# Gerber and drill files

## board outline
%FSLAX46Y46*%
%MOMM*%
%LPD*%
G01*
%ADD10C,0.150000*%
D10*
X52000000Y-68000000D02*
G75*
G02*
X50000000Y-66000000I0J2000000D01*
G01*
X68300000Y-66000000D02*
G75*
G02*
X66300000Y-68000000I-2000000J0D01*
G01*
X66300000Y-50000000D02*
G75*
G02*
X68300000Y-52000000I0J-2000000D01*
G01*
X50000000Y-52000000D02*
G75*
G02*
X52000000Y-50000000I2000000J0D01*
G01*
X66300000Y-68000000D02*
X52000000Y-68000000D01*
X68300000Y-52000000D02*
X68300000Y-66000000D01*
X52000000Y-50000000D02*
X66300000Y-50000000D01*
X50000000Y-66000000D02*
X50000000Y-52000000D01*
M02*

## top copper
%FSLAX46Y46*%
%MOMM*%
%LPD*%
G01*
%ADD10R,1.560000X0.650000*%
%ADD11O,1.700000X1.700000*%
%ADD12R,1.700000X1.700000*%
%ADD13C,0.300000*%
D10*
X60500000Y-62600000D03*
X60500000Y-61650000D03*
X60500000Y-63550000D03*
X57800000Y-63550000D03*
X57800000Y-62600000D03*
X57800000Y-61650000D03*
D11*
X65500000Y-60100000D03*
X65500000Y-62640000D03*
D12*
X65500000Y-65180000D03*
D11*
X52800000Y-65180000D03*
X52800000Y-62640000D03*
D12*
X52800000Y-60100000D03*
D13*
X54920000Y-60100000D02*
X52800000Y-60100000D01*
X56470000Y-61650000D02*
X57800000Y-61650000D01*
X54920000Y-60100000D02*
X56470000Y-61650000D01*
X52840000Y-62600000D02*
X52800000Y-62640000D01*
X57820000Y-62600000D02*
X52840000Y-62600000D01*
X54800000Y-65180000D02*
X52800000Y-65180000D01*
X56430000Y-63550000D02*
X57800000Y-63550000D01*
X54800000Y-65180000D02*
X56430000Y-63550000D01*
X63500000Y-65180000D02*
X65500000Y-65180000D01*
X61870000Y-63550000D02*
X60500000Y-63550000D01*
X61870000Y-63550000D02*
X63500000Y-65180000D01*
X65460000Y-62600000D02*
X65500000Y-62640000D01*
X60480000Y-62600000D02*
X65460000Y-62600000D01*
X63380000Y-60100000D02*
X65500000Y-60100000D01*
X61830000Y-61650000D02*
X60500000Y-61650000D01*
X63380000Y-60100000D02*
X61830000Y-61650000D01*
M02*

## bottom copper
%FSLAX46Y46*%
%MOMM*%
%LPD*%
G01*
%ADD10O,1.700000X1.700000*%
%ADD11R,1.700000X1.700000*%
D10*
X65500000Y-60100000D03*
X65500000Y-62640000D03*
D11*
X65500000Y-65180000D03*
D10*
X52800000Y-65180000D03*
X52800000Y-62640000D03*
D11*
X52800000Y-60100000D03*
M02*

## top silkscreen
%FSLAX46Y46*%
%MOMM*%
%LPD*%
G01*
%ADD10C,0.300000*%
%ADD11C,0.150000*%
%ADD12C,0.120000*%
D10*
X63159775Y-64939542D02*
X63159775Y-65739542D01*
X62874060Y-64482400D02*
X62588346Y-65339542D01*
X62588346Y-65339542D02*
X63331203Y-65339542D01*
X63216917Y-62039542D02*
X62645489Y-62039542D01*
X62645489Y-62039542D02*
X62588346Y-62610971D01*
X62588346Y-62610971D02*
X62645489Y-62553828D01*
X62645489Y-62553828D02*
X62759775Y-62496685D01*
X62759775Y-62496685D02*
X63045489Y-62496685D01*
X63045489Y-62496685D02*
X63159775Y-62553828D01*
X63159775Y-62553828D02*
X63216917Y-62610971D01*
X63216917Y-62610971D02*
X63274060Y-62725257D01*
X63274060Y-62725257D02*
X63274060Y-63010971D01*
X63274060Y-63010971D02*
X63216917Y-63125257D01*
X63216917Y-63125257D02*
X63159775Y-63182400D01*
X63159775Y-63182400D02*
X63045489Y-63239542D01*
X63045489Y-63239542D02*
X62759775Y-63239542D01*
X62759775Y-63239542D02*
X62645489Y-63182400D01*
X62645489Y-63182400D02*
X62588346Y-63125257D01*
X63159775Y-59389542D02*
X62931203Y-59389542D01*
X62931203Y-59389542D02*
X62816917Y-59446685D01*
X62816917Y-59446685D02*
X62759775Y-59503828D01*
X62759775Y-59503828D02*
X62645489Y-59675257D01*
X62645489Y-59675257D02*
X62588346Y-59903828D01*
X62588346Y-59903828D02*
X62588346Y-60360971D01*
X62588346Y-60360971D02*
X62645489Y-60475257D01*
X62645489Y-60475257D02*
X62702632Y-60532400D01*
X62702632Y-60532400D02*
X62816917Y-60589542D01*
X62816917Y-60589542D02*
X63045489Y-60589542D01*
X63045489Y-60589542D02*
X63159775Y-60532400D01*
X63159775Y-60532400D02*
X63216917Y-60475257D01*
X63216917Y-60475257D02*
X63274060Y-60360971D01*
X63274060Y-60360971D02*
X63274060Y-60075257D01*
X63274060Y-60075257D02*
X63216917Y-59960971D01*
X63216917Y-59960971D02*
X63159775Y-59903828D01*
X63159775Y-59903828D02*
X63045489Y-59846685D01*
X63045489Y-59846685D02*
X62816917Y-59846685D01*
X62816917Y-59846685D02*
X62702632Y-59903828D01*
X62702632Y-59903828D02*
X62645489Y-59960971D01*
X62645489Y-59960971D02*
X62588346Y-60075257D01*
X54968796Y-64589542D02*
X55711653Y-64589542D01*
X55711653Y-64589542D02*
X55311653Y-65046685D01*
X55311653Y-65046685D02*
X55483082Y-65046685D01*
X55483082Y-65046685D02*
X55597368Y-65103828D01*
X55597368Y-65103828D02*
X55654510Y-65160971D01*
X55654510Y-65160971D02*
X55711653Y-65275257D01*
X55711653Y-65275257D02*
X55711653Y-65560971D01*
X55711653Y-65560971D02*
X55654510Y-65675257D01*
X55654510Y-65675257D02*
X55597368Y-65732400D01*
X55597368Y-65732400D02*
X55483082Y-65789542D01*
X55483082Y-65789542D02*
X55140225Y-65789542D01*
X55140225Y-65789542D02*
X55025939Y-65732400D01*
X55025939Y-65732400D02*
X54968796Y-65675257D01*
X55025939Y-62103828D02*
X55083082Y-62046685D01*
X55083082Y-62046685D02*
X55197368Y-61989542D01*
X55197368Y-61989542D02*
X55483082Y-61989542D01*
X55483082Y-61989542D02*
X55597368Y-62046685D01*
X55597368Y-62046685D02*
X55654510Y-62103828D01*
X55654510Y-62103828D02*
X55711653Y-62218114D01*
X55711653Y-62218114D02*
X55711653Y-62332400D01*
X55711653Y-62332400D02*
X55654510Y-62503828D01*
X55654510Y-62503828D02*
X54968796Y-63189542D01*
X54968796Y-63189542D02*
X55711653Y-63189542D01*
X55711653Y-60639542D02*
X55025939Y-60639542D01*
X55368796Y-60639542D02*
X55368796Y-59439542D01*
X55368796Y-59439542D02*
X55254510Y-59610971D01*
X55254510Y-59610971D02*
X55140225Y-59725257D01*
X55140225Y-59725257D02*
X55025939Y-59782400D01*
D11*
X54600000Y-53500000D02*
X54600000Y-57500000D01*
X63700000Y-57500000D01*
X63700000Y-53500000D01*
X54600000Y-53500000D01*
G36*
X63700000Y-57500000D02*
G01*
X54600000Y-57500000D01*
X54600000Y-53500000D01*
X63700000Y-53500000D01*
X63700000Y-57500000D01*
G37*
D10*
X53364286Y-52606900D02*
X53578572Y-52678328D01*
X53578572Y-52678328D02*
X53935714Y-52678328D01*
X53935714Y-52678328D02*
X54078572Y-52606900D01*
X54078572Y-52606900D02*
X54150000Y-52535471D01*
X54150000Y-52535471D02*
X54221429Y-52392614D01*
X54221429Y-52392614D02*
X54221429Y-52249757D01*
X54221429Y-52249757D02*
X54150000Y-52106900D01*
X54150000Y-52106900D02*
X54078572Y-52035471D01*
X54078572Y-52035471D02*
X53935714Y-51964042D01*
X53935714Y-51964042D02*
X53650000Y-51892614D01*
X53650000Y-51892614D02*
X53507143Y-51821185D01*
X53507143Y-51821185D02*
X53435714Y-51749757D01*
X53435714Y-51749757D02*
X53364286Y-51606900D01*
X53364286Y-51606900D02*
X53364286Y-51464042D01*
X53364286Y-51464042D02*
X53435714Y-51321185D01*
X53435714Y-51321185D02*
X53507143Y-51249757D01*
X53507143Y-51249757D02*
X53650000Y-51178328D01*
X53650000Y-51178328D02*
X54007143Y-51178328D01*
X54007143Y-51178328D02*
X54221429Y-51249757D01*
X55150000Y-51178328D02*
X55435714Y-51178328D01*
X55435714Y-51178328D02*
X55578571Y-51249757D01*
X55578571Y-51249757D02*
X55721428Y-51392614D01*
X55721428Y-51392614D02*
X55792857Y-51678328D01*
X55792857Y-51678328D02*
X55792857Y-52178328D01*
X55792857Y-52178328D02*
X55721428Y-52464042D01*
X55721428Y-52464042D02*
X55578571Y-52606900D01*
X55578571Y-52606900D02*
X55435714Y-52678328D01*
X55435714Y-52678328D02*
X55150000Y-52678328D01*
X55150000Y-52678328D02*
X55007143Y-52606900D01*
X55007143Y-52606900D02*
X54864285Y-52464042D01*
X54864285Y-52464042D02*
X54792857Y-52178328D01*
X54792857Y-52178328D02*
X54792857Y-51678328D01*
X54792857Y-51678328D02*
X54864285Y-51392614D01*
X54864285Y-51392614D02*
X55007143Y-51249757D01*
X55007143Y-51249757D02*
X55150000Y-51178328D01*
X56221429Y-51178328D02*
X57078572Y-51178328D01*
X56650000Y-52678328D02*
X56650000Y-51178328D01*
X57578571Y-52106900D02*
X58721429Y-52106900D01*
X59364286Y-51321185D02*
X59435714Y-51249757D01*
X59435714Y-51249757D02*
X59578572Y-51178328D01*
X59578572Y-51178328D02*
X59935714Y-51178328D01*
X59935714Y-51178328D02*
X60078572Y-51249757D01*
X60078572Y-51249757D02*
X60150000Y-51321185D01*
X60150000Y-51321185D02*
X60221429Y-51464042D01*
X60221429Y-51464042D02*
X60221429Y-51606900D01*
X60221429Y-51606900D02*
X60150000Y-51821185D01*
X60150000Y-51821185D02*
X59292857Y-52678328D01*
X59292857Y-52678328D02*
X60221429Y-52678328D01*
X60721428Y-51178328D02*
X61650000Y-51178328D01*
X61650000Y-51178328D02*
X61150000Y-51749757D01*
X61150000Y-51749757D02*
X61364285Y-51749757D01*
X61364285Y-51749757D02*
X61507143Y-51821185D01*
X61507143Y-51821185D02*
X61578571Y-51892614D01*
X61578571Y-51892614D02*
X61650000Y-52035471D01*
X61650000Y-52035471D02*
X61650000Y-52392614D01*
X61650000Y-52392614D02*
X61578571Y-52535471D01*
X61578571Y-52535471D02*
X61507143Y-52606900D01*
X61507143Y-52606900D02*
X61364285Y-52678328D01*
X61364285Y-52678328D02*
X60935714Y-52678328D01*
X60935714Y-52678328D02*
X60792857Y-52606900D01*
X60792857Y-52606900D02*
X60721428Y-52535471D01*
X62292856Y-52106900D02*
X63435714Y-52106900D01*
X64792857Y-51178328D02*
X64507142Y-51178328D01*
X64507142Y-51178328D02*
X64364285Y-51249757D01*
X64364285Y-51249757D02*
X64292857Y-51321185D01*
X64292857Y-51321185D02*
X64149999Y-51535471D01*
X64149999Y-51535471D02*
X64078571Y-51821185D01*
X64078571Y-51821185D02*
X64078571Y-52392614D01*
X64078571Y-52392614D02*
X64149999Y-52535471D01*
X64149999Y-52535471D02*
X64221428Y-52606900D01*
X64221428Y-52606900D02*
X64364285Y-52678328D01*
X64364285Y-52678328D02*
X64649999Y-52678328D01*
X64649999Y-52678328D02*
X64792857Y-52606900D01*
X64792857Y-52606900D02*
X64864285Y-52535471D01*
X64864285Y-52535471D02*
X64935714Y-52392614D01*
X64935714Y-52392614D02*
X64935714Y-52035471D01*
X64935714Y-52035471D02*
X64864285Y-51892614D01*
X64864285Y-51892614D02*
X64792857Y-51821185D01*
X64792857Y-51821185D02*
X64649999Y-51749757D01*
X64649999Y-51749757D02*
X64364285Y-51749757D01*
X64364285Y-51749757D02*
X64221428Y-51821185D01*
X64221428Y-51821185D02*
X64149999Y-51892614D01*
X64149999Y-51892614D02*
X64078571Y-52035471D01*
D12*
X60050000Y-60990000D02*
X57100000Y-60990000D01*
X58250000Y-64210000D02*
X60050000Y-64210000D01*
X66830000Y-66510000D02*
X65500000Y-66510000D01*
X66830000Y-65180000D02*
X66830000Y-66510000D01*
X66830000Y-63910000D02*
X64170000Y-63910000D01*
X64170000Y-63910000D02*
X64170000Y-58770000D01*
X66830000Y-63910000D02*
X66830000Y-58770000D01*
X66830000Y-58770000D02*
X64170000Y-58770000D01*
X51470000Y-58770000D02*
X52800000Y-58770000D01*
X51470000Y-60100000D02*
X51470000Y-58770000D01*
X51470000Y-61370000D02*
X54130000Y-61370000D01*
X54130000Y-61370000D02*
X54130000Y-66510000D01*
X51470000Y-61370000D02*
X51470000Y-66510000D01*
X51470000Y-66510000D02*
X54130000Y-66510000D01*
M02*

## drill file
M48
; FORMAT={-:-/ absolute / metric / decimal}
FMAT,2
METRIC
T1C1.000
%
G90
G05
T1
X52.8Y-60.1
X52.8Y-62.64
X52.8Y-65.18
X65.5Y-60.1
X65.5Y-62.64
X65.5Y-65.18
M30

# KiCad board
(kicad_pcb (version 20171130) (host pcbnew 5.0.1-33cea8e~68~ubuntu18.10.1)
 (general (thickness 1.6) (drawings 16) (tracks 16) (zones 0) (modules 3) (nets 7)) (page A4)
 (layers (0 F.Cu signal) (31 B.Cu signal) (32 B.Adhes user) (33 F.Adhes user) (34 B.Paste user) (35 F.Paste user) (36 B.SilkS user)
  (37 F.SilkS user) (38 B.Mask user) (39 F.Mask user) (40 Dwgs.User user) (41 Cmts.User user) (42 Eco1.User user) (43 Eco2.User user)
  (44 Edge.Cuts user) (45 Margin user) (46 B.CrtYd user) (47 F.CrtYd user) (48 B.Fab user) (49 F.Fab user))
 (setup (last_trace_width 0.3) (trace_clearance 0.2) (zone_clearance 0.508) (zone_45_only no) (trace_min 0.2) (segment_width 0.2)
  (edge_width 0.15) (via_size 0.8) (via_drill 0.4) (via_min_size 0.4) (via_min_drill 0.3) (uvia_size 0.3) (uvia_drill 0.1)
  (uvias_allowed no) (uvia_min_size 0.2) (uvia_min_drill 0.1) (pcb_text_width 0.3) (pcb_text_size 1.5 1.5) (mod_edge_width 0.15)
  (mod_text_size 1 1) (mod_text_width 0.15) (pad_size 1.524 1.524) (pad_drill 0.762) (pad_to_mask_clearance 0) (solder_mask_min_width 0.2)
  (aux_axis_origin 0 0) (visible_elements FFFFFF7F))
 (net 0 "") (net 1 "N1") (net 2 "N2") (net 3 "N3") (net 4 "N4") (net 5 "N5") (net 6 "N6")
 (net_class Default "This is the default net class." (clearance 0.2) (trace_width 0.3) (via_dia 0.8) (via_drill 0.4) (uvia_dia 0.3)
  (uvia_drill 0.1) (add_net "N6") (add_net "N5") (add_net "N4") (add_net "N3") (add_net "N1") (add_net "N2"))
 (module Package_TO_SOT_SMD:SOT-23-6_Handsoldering (layer F.Cu) (at 59.15 62.6)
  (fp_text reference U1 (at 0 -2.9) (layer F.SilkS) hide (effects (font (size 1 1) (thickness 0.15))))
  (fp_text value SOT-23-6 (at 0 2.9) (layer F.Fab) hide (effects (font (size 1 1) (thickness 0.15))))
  (fp_line (start 0.9 -1.61) (end -2.05 -1.61) (layer F.SilkS) (width 0.12))
  (fp_line (start -0.9 1.61) (end 0.9 1.61) (layer F.SilkS) (width 0.12))
  (pad 5 smd rect (at 1.35 0) (size 1.56 0.65) (layers F.Cu F.Paste F.Mask) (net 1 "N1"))
  (pad 6 smd rect (at 1.35 -0.95) (size 1.56 0.65) (layers F.Cu F.Paste F.Mask) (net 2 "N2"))
  (pad 4 smd rect (at 1.35 0.95) (size 1.56 0.65) (layers F.Cu F.Paste F.Mask) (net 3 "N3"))
  (pad 3 smd rect (at -1.35 0.95) (size 1.56 0.65) (layers F.Cu F.Paste F.Mask) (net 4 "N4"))
  (pad 2 smd rect (at -1.35 0) (size 1.56 0.65) (layers F.Cu F.Paste F.Mask) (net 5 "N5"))
  (pad 1 smd rect (at -1.35 -0.95) (size 1.56 0.65) (layers F.Cu F.Paste F.Mask) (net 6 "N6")))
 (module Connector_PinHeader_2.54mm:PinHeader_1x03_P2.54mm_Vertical (layer F.Cu) (at 65.5 65.18 180)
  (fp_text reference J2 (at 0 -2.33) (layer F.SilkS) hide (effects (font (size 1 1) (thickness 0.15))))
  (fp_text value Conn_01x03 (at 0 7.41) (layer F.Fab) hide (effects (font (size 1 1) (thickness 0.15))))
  (fp_line (start -1.33 -1.33) (end 0 -1.33) (layer F.SilkS) (width 0.12))
  (fp_line (start -1.33 0) (end -1.33 -1.33) (layer F.SilkS) (width 0.12))
  (fp_line (start -1.33 1.27) (end 1.33 1.27) (layer F.SilkS) (width 0.12))
  (fp_line (start 1.33 1.27) (end 1.33 6.41) (layer F.SilkS) (width 0.12))
  (fp_line (start -1.33 1.27) (end -1.33 6.41) (layer F.SilkS) (width 0.12))
  (fp_line (start -1.33 6.41) (end 1.33 6.41) (layer F.SilkS) (width 0.12))
  (pad 3 thru_hole oval (at 0 5.08 180) (size 1.7 1.7) (drill 1) (layers *.Cu *.Mask) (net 2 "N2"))
  (pad 2 thru_hole oval (at 0 2.54 180) (size 1.7 1.7) (drill 1) (layers *.Cu *.Mask) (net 1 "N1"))
  (pad 1 thru_hole rect (at 0 0 180) (size 1.7 1.7) (drill 1) (layers *.Cu *.Mask) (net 3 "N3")))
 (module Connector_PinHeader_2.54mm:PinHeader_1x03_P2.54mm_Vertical (layer F.Cu) (at 52.8 60.1)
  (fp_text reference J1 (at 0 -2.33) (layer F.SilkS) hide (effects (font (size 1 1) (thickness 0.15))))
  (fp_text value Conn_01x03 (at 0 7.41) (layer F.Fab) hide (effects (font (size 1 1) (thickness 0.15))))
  (fp_line (start -1.33 -1.33) (end 0 -1.33) (layer F.SilkS) (width 0.12))
  (fp_line (start -1.33 0) (end -1.33 -1.33) (layer F.SilkS) (width 0.12))
  (fp_line (start -1.33 1.27) (end 1.33 1.27) (layer F.SilkS) (width 0.12))
  (fp_line (start 1.33 1.27) (end 1.33 6.41) (layer F.SilkS) (width 0.12))
  (fp_line (start -1.33 1.27) (end -1.33 6.41) (layer F.SilkS) (width 0.12))
  (fp_line (start -1.33 6.41) (end 1.33 6.41) (layer F.SilkS) (width 0.12))
  (pad 3 thru_hole oval (at 0 5.08) (size 1.7 1.7) (drill 1) (layers *.Cu *.Mask) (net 4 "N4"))
  (pad 2 thru_hole oval (at 0 2.54) (size 1.7 1.7) (drill 1) (layers *.Cu *.Mask) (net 5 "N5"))
  (pad 1 thru_hole rect (at 0 0) (size 1.7 1.7) (drill 1) (layers *.Cu *.Mask) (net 6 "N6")))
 (gr_arc (start 52 66) (end 50 66) (angle -90) (layer Edge.Cuts) (width 0.15))
 (gr_arc (start 66.3 66) (end 66.3 68) (angle -90) (layer Edge.Cuts) (width 0.15))
 (gr_arc (start 66.3 52) (end 68.3 52) (angle -90) (layer Edge.Cuts) (width 0.15))
 (gr_arc (start 52 52) (end 52 50) (angle -90) (layer Edge.Cuts) (width 0.15))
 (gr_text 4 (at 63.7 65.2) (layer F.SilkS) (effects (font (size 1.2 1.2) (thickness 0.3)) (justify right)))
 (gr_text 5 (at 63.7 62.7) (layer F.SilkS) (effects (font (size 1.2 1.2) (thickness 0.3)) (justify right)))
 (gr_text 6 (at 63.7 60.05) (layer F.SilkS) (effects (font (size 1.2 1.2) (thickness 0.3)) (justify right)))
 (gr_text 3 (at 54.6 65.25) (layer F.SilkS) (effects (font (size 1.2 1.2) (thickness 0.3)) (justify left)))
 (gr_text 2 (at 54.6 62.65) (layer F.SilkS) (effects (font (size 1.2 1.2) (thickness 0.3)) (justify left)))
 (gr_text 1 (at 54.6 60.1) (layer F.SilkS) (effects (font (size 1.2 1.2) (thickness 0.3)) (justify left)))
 (gr_line (start 66.3 68) (end 52 68) (layer Edge.Cuts) (width 0.15))
 (gr_poly (pts (xy 54.6 53.5) (xy 54.6 57.5) (xy 63.7 57.5) (xy 63.7 53.5)) (layer F.SilkS) (width 0.15))
 (gr_line (start 68.3 52) (end 68.3 66) (layer Edge.Cuts) (width 0.15))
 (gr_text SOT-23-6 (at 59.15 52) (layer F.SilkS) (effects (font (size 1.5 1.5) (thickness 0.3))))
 (gr_line (start 52 50) (end 66.3 50) (layer Edge.Cuts) (width 0.15))
 (gr_line (start 50 66) (end 50 52) (layer Edge.Cuts) (width 0.15))
 (segment (start 54.92 60.1) (end 52.8 60.1) (width 0.3) (layer F.Cu) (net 6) (status 20))
 (segment (start 56.47 61.65) (end 57.8 61.65) (width 0.3) (layer F.Cu) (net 6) (status 20))
 (segment (start 54.92 60.1) (end 56.47 61.65) (width 0.3) (layer F.Cu) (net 6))
 (segment (start 52.84 62.6) (end 52.8 62.64) (width 0.3) (layer F.Cu) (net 5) (status 30))
 (segment (start 57.82 62.6) (end 52.84 62.6) (width 0.3) (layer F.Cu) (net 5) (status 30))
 (segment (start 54.8 65.18) (end 52.8 65.18) (width 0.3) (layer F.Cu) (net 4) (status 20))
 (segment (start 56.43 63.55) (end 57.8 63.55) (width 0.3) (layer F.Cu) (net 4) (status 20))
 (segment (start 54.8 65.18) (end 56.43 63.55) (width 0.3) (layer F.Cu) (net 4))
 (segment (start 63.5 65.18) (end 65.5 65.18) (width 0.3) (layer F.Cu) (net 3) (status 20))
 (segment (start 61.87 63.55) (end 60.5 63.55) (width 0.3) (layer F.Cu) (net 3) (status 20))
 (segment (start 61.87 63.55) (end 63.5 65.18) (width 0.3) (layer F.Cu) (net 3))
 (segment (start 65.46 62.6) (end 65.5 62.64) (width 0.3) (layer F.Cu) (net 1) (status 30))
 (segment (start 60.48 62.6) (end 65.46 62.6) (width 0.3) (layer F.Cu) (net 1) (status 30))
 (segment (start 63.38 60.1) (end 65.5 60.1) (width 0.3) (layer F.Cu) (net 2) (status 20))
 (segment (start 61.83 61.65) (end 60.5 61.65) (width 0.3) (layer F.Cu) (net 2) (status 20))
 (segment (start 63.38 60.1) (end 61.83 61.65) (width 0.3) (layer F.Cu) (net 2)))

